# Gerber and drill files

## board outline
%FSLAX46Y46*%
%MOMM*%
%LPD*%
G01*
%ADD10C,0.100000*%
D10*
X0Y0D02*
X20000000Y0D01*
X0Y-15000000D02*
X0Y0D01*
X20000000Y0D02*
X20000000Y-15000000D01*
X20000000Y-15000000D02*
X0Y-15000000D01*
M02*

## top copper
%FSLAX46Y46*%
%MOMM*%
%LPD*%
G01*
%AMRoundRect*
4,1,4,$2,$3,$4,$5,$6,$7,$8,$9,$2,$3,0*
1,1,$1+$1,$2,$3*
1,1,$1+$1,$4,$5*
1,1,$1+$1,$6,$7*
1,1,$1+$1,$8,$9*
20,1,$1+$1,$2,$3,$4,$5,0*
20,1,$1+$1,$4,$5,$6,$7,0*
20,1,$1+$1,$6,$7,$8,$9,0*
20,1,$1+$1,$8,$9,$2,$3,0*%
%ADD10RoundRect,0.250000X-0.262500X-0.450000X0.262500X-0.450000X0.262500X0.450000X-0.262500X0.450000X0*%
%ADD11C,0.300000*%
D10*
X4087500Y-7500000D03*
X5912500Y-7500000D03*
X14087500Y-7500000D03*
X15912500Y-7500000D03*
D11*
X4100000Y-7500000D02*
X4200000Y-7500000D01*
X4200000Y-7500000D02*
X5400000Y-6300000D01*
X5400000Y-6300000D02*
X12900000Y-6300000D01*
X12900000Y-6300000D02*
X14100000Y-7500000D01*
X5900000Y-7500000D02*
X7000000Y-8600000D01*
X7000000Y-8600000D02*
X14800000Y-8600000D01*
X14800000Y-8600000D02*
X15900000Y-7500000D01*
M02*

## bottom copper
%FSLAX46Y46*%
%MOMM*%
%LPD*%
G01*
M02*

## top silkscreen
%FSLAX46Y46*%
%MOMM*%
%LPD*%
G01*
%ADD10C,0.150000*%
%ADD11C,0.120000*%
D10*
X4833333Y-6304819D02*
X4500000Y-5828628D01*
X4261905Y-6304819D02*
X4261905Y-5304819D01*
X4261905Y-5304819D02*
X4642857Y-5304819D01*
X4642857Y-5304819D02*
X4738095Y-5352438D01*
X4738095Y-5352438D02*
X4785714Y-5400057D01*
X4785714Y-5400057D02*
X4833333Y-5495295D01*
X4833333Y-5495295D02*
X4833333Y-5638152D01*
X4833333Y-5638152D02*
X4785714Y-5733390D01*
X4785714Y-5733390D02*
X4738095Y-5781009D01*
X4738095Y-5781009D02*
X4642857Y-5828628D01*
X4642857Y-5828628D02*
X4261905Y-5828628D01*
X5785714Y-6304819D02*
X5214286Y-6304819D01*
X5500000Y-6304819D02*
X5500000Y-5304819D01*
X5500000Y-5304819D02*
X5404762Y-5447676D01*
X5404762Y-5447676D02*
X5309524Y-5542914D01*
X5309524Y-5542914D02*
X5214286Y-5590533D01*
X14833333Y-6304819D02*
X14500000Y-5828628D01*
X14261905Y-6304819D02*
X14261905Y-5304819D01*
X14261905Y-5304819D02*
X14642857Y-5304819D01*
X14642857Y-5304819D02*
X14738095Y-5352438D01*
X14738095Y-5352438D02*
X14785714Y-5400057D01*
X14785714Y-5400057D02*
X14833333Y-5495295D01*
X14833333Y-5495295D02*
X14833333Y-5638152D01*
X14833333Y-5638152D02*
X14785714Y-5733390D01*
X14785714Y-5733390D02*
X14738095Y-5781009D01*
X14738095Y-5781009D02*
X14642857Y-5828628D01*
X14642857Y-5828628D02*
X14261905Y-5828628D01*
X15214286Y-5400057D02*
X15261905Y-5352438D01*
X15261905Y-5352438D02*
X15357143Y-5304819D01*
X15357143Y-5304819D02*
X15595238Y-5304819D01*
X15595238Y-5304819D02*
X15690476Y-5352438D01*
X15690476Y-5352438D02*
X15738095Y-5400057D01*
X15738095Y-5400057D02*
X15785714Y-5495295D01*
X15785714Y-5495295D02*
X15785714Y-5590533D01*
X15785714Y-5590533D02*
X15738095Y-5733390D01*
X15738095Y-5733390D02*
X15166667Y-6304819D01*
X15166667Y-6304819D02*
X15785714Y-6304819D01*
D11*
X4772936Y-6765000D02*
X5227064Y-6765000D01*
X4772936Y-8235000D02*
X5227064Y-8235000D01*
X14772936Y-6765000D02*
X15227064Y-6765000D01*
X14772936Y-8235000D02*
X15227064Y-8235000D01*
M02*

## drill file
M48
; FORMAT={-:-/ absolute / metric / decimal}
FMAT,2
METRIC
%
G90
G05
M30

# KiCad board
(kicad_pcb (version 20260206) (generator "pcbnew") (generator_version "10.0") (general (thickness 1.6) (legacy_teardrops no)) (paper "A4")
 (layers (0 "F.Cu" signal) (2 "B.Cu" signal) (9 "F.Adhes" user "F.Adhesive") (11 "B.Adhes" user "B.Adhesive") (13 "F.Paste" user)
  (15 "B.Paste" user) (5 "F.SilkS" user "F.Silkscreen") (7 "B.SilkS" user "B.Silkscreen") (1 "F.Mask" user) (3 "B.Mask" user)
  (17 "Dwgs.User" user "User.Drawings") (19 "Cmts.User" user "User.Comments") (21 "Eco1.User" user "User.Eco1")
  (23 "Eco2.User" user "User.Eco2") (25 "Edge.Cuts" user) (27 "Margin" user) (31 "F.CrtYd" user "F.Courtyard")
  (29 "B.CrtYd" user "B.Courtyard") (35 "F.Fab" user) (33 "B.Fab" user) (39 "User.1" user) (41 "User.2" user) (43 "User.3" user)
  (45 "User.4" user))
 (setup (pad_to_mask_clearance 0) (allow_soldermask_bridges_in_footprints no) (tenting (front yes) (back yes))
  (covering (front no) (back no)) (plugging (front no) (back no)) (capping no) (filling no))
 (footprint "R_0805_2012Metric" (layer "F.Cu") (at 5 7.5)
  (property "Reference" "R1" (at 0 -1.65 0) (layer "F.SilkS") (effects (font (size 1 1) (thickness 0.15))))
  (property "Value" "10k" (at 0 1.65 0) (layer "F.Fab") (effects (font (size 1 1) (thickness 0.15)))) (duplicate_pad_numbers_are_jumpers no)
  (fp_line (start -0.227064 -0.735) (end 0.227064 -0.735) (stroke (width 0.12) (type solid)) (layer "F.SilkS"))
  (fp_line (start -0.227064 0.735) (end 0.227064 0.735) (stroke (width 0.12) (type solid)) (layer "F.SilkS"))
  (pad "1" smd roundrect (at -0.9125 0) (size 1.025 1.4) (layers "F.Cu" "F.Mask" "F.Paste") (roundrect_rratio 0.243902) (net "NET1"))
  (pad "2" smd roundrect (at 0.9125 0) (size 1.025 1.4) (layers "F.Cu" "F.Mask" "F.Paste") (roundrect_rratio 0.243902) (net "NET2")))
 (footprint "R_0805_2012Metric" (layer "F.Cu") (at 15 7.5)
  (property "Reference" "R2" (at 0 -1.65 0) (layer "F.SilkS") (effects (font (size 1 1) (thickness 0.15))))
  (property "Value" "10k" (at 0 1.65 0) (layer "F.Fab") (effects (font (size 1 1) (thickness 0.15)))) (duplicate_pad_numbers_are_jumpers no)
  (fp_line (start -0.227064 -0.735) (end 0.227064 -0.735) (stroke (width 0.12) (type solid)) (layer "F.SilkS"))
  (fp_line (start -0.227064 0.735) (end 0.227064 0.735) (stroke (width 0.12) (type solid)) (layer "F.SilkS"))
  (pad "1" smd roundrect (at -0.9125 0) (size 1.025 1.4) (layers "F.Cu" "F.Mask" "F.Paste") (roundrect_rratio 0.243902) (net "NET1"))
  (pad "2" smd roundrect (at 0.9125 0) (size 1.025 1.4) (layers "F.Cu" "F.Mask" "F.Paste") (roundrect_rratio 0.243902) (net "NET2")))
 (gr_line (start 0 0) (end 20 0) (stroke (width 0.1) (type default)) (layer "Edge.Cuts"))
 (gr_line (start 0 15) (end 0 0) (stroke (width 0.1) (type default)) (layer "Edge.Cuts"))
 (gr_line (start 20 0) (end 20 15) (stroke (width 0.1) (type default)) (layer "Edge.Cuts"))
 (gr_line (start 20 15) (end 0 15) (stroke (width 0.1) (type default)) (layer "Edge.Cuts"))
 (segment (start 4.100000 7.500000) (end 4.200000 7.500000) (width 0.3) (layer "F.Cu") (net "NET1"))
 (segment (start 4.200000 7.500000) (end 5.400000 6.300000) (width 0.3) (layer "F.Cu") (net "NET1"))
 (segment (start 5.400000 6.300000) (end 12.900000 6.300000) (width 0.3) (layer "F.Cu") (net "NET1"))
 (segment (start 12.900000 6.300000) (end 14.100000 7.500000) (width 0.3) (layer "F.Cu") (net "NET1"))
 (segment (start 5.900000 7.500000) (end 7.000000 8.600000) (width 0.3) (layer "F.Cu") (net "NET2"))
 (segment (start 7.000000 8.600000) (end 14.800000 8.600000) (width 0.3) (layer "F.Cu") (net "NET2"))
 (segment (start 14.800000 8.600000) (end 15.900000 7.500000) (width 0.3) (layer "F.Cu") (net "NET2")))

